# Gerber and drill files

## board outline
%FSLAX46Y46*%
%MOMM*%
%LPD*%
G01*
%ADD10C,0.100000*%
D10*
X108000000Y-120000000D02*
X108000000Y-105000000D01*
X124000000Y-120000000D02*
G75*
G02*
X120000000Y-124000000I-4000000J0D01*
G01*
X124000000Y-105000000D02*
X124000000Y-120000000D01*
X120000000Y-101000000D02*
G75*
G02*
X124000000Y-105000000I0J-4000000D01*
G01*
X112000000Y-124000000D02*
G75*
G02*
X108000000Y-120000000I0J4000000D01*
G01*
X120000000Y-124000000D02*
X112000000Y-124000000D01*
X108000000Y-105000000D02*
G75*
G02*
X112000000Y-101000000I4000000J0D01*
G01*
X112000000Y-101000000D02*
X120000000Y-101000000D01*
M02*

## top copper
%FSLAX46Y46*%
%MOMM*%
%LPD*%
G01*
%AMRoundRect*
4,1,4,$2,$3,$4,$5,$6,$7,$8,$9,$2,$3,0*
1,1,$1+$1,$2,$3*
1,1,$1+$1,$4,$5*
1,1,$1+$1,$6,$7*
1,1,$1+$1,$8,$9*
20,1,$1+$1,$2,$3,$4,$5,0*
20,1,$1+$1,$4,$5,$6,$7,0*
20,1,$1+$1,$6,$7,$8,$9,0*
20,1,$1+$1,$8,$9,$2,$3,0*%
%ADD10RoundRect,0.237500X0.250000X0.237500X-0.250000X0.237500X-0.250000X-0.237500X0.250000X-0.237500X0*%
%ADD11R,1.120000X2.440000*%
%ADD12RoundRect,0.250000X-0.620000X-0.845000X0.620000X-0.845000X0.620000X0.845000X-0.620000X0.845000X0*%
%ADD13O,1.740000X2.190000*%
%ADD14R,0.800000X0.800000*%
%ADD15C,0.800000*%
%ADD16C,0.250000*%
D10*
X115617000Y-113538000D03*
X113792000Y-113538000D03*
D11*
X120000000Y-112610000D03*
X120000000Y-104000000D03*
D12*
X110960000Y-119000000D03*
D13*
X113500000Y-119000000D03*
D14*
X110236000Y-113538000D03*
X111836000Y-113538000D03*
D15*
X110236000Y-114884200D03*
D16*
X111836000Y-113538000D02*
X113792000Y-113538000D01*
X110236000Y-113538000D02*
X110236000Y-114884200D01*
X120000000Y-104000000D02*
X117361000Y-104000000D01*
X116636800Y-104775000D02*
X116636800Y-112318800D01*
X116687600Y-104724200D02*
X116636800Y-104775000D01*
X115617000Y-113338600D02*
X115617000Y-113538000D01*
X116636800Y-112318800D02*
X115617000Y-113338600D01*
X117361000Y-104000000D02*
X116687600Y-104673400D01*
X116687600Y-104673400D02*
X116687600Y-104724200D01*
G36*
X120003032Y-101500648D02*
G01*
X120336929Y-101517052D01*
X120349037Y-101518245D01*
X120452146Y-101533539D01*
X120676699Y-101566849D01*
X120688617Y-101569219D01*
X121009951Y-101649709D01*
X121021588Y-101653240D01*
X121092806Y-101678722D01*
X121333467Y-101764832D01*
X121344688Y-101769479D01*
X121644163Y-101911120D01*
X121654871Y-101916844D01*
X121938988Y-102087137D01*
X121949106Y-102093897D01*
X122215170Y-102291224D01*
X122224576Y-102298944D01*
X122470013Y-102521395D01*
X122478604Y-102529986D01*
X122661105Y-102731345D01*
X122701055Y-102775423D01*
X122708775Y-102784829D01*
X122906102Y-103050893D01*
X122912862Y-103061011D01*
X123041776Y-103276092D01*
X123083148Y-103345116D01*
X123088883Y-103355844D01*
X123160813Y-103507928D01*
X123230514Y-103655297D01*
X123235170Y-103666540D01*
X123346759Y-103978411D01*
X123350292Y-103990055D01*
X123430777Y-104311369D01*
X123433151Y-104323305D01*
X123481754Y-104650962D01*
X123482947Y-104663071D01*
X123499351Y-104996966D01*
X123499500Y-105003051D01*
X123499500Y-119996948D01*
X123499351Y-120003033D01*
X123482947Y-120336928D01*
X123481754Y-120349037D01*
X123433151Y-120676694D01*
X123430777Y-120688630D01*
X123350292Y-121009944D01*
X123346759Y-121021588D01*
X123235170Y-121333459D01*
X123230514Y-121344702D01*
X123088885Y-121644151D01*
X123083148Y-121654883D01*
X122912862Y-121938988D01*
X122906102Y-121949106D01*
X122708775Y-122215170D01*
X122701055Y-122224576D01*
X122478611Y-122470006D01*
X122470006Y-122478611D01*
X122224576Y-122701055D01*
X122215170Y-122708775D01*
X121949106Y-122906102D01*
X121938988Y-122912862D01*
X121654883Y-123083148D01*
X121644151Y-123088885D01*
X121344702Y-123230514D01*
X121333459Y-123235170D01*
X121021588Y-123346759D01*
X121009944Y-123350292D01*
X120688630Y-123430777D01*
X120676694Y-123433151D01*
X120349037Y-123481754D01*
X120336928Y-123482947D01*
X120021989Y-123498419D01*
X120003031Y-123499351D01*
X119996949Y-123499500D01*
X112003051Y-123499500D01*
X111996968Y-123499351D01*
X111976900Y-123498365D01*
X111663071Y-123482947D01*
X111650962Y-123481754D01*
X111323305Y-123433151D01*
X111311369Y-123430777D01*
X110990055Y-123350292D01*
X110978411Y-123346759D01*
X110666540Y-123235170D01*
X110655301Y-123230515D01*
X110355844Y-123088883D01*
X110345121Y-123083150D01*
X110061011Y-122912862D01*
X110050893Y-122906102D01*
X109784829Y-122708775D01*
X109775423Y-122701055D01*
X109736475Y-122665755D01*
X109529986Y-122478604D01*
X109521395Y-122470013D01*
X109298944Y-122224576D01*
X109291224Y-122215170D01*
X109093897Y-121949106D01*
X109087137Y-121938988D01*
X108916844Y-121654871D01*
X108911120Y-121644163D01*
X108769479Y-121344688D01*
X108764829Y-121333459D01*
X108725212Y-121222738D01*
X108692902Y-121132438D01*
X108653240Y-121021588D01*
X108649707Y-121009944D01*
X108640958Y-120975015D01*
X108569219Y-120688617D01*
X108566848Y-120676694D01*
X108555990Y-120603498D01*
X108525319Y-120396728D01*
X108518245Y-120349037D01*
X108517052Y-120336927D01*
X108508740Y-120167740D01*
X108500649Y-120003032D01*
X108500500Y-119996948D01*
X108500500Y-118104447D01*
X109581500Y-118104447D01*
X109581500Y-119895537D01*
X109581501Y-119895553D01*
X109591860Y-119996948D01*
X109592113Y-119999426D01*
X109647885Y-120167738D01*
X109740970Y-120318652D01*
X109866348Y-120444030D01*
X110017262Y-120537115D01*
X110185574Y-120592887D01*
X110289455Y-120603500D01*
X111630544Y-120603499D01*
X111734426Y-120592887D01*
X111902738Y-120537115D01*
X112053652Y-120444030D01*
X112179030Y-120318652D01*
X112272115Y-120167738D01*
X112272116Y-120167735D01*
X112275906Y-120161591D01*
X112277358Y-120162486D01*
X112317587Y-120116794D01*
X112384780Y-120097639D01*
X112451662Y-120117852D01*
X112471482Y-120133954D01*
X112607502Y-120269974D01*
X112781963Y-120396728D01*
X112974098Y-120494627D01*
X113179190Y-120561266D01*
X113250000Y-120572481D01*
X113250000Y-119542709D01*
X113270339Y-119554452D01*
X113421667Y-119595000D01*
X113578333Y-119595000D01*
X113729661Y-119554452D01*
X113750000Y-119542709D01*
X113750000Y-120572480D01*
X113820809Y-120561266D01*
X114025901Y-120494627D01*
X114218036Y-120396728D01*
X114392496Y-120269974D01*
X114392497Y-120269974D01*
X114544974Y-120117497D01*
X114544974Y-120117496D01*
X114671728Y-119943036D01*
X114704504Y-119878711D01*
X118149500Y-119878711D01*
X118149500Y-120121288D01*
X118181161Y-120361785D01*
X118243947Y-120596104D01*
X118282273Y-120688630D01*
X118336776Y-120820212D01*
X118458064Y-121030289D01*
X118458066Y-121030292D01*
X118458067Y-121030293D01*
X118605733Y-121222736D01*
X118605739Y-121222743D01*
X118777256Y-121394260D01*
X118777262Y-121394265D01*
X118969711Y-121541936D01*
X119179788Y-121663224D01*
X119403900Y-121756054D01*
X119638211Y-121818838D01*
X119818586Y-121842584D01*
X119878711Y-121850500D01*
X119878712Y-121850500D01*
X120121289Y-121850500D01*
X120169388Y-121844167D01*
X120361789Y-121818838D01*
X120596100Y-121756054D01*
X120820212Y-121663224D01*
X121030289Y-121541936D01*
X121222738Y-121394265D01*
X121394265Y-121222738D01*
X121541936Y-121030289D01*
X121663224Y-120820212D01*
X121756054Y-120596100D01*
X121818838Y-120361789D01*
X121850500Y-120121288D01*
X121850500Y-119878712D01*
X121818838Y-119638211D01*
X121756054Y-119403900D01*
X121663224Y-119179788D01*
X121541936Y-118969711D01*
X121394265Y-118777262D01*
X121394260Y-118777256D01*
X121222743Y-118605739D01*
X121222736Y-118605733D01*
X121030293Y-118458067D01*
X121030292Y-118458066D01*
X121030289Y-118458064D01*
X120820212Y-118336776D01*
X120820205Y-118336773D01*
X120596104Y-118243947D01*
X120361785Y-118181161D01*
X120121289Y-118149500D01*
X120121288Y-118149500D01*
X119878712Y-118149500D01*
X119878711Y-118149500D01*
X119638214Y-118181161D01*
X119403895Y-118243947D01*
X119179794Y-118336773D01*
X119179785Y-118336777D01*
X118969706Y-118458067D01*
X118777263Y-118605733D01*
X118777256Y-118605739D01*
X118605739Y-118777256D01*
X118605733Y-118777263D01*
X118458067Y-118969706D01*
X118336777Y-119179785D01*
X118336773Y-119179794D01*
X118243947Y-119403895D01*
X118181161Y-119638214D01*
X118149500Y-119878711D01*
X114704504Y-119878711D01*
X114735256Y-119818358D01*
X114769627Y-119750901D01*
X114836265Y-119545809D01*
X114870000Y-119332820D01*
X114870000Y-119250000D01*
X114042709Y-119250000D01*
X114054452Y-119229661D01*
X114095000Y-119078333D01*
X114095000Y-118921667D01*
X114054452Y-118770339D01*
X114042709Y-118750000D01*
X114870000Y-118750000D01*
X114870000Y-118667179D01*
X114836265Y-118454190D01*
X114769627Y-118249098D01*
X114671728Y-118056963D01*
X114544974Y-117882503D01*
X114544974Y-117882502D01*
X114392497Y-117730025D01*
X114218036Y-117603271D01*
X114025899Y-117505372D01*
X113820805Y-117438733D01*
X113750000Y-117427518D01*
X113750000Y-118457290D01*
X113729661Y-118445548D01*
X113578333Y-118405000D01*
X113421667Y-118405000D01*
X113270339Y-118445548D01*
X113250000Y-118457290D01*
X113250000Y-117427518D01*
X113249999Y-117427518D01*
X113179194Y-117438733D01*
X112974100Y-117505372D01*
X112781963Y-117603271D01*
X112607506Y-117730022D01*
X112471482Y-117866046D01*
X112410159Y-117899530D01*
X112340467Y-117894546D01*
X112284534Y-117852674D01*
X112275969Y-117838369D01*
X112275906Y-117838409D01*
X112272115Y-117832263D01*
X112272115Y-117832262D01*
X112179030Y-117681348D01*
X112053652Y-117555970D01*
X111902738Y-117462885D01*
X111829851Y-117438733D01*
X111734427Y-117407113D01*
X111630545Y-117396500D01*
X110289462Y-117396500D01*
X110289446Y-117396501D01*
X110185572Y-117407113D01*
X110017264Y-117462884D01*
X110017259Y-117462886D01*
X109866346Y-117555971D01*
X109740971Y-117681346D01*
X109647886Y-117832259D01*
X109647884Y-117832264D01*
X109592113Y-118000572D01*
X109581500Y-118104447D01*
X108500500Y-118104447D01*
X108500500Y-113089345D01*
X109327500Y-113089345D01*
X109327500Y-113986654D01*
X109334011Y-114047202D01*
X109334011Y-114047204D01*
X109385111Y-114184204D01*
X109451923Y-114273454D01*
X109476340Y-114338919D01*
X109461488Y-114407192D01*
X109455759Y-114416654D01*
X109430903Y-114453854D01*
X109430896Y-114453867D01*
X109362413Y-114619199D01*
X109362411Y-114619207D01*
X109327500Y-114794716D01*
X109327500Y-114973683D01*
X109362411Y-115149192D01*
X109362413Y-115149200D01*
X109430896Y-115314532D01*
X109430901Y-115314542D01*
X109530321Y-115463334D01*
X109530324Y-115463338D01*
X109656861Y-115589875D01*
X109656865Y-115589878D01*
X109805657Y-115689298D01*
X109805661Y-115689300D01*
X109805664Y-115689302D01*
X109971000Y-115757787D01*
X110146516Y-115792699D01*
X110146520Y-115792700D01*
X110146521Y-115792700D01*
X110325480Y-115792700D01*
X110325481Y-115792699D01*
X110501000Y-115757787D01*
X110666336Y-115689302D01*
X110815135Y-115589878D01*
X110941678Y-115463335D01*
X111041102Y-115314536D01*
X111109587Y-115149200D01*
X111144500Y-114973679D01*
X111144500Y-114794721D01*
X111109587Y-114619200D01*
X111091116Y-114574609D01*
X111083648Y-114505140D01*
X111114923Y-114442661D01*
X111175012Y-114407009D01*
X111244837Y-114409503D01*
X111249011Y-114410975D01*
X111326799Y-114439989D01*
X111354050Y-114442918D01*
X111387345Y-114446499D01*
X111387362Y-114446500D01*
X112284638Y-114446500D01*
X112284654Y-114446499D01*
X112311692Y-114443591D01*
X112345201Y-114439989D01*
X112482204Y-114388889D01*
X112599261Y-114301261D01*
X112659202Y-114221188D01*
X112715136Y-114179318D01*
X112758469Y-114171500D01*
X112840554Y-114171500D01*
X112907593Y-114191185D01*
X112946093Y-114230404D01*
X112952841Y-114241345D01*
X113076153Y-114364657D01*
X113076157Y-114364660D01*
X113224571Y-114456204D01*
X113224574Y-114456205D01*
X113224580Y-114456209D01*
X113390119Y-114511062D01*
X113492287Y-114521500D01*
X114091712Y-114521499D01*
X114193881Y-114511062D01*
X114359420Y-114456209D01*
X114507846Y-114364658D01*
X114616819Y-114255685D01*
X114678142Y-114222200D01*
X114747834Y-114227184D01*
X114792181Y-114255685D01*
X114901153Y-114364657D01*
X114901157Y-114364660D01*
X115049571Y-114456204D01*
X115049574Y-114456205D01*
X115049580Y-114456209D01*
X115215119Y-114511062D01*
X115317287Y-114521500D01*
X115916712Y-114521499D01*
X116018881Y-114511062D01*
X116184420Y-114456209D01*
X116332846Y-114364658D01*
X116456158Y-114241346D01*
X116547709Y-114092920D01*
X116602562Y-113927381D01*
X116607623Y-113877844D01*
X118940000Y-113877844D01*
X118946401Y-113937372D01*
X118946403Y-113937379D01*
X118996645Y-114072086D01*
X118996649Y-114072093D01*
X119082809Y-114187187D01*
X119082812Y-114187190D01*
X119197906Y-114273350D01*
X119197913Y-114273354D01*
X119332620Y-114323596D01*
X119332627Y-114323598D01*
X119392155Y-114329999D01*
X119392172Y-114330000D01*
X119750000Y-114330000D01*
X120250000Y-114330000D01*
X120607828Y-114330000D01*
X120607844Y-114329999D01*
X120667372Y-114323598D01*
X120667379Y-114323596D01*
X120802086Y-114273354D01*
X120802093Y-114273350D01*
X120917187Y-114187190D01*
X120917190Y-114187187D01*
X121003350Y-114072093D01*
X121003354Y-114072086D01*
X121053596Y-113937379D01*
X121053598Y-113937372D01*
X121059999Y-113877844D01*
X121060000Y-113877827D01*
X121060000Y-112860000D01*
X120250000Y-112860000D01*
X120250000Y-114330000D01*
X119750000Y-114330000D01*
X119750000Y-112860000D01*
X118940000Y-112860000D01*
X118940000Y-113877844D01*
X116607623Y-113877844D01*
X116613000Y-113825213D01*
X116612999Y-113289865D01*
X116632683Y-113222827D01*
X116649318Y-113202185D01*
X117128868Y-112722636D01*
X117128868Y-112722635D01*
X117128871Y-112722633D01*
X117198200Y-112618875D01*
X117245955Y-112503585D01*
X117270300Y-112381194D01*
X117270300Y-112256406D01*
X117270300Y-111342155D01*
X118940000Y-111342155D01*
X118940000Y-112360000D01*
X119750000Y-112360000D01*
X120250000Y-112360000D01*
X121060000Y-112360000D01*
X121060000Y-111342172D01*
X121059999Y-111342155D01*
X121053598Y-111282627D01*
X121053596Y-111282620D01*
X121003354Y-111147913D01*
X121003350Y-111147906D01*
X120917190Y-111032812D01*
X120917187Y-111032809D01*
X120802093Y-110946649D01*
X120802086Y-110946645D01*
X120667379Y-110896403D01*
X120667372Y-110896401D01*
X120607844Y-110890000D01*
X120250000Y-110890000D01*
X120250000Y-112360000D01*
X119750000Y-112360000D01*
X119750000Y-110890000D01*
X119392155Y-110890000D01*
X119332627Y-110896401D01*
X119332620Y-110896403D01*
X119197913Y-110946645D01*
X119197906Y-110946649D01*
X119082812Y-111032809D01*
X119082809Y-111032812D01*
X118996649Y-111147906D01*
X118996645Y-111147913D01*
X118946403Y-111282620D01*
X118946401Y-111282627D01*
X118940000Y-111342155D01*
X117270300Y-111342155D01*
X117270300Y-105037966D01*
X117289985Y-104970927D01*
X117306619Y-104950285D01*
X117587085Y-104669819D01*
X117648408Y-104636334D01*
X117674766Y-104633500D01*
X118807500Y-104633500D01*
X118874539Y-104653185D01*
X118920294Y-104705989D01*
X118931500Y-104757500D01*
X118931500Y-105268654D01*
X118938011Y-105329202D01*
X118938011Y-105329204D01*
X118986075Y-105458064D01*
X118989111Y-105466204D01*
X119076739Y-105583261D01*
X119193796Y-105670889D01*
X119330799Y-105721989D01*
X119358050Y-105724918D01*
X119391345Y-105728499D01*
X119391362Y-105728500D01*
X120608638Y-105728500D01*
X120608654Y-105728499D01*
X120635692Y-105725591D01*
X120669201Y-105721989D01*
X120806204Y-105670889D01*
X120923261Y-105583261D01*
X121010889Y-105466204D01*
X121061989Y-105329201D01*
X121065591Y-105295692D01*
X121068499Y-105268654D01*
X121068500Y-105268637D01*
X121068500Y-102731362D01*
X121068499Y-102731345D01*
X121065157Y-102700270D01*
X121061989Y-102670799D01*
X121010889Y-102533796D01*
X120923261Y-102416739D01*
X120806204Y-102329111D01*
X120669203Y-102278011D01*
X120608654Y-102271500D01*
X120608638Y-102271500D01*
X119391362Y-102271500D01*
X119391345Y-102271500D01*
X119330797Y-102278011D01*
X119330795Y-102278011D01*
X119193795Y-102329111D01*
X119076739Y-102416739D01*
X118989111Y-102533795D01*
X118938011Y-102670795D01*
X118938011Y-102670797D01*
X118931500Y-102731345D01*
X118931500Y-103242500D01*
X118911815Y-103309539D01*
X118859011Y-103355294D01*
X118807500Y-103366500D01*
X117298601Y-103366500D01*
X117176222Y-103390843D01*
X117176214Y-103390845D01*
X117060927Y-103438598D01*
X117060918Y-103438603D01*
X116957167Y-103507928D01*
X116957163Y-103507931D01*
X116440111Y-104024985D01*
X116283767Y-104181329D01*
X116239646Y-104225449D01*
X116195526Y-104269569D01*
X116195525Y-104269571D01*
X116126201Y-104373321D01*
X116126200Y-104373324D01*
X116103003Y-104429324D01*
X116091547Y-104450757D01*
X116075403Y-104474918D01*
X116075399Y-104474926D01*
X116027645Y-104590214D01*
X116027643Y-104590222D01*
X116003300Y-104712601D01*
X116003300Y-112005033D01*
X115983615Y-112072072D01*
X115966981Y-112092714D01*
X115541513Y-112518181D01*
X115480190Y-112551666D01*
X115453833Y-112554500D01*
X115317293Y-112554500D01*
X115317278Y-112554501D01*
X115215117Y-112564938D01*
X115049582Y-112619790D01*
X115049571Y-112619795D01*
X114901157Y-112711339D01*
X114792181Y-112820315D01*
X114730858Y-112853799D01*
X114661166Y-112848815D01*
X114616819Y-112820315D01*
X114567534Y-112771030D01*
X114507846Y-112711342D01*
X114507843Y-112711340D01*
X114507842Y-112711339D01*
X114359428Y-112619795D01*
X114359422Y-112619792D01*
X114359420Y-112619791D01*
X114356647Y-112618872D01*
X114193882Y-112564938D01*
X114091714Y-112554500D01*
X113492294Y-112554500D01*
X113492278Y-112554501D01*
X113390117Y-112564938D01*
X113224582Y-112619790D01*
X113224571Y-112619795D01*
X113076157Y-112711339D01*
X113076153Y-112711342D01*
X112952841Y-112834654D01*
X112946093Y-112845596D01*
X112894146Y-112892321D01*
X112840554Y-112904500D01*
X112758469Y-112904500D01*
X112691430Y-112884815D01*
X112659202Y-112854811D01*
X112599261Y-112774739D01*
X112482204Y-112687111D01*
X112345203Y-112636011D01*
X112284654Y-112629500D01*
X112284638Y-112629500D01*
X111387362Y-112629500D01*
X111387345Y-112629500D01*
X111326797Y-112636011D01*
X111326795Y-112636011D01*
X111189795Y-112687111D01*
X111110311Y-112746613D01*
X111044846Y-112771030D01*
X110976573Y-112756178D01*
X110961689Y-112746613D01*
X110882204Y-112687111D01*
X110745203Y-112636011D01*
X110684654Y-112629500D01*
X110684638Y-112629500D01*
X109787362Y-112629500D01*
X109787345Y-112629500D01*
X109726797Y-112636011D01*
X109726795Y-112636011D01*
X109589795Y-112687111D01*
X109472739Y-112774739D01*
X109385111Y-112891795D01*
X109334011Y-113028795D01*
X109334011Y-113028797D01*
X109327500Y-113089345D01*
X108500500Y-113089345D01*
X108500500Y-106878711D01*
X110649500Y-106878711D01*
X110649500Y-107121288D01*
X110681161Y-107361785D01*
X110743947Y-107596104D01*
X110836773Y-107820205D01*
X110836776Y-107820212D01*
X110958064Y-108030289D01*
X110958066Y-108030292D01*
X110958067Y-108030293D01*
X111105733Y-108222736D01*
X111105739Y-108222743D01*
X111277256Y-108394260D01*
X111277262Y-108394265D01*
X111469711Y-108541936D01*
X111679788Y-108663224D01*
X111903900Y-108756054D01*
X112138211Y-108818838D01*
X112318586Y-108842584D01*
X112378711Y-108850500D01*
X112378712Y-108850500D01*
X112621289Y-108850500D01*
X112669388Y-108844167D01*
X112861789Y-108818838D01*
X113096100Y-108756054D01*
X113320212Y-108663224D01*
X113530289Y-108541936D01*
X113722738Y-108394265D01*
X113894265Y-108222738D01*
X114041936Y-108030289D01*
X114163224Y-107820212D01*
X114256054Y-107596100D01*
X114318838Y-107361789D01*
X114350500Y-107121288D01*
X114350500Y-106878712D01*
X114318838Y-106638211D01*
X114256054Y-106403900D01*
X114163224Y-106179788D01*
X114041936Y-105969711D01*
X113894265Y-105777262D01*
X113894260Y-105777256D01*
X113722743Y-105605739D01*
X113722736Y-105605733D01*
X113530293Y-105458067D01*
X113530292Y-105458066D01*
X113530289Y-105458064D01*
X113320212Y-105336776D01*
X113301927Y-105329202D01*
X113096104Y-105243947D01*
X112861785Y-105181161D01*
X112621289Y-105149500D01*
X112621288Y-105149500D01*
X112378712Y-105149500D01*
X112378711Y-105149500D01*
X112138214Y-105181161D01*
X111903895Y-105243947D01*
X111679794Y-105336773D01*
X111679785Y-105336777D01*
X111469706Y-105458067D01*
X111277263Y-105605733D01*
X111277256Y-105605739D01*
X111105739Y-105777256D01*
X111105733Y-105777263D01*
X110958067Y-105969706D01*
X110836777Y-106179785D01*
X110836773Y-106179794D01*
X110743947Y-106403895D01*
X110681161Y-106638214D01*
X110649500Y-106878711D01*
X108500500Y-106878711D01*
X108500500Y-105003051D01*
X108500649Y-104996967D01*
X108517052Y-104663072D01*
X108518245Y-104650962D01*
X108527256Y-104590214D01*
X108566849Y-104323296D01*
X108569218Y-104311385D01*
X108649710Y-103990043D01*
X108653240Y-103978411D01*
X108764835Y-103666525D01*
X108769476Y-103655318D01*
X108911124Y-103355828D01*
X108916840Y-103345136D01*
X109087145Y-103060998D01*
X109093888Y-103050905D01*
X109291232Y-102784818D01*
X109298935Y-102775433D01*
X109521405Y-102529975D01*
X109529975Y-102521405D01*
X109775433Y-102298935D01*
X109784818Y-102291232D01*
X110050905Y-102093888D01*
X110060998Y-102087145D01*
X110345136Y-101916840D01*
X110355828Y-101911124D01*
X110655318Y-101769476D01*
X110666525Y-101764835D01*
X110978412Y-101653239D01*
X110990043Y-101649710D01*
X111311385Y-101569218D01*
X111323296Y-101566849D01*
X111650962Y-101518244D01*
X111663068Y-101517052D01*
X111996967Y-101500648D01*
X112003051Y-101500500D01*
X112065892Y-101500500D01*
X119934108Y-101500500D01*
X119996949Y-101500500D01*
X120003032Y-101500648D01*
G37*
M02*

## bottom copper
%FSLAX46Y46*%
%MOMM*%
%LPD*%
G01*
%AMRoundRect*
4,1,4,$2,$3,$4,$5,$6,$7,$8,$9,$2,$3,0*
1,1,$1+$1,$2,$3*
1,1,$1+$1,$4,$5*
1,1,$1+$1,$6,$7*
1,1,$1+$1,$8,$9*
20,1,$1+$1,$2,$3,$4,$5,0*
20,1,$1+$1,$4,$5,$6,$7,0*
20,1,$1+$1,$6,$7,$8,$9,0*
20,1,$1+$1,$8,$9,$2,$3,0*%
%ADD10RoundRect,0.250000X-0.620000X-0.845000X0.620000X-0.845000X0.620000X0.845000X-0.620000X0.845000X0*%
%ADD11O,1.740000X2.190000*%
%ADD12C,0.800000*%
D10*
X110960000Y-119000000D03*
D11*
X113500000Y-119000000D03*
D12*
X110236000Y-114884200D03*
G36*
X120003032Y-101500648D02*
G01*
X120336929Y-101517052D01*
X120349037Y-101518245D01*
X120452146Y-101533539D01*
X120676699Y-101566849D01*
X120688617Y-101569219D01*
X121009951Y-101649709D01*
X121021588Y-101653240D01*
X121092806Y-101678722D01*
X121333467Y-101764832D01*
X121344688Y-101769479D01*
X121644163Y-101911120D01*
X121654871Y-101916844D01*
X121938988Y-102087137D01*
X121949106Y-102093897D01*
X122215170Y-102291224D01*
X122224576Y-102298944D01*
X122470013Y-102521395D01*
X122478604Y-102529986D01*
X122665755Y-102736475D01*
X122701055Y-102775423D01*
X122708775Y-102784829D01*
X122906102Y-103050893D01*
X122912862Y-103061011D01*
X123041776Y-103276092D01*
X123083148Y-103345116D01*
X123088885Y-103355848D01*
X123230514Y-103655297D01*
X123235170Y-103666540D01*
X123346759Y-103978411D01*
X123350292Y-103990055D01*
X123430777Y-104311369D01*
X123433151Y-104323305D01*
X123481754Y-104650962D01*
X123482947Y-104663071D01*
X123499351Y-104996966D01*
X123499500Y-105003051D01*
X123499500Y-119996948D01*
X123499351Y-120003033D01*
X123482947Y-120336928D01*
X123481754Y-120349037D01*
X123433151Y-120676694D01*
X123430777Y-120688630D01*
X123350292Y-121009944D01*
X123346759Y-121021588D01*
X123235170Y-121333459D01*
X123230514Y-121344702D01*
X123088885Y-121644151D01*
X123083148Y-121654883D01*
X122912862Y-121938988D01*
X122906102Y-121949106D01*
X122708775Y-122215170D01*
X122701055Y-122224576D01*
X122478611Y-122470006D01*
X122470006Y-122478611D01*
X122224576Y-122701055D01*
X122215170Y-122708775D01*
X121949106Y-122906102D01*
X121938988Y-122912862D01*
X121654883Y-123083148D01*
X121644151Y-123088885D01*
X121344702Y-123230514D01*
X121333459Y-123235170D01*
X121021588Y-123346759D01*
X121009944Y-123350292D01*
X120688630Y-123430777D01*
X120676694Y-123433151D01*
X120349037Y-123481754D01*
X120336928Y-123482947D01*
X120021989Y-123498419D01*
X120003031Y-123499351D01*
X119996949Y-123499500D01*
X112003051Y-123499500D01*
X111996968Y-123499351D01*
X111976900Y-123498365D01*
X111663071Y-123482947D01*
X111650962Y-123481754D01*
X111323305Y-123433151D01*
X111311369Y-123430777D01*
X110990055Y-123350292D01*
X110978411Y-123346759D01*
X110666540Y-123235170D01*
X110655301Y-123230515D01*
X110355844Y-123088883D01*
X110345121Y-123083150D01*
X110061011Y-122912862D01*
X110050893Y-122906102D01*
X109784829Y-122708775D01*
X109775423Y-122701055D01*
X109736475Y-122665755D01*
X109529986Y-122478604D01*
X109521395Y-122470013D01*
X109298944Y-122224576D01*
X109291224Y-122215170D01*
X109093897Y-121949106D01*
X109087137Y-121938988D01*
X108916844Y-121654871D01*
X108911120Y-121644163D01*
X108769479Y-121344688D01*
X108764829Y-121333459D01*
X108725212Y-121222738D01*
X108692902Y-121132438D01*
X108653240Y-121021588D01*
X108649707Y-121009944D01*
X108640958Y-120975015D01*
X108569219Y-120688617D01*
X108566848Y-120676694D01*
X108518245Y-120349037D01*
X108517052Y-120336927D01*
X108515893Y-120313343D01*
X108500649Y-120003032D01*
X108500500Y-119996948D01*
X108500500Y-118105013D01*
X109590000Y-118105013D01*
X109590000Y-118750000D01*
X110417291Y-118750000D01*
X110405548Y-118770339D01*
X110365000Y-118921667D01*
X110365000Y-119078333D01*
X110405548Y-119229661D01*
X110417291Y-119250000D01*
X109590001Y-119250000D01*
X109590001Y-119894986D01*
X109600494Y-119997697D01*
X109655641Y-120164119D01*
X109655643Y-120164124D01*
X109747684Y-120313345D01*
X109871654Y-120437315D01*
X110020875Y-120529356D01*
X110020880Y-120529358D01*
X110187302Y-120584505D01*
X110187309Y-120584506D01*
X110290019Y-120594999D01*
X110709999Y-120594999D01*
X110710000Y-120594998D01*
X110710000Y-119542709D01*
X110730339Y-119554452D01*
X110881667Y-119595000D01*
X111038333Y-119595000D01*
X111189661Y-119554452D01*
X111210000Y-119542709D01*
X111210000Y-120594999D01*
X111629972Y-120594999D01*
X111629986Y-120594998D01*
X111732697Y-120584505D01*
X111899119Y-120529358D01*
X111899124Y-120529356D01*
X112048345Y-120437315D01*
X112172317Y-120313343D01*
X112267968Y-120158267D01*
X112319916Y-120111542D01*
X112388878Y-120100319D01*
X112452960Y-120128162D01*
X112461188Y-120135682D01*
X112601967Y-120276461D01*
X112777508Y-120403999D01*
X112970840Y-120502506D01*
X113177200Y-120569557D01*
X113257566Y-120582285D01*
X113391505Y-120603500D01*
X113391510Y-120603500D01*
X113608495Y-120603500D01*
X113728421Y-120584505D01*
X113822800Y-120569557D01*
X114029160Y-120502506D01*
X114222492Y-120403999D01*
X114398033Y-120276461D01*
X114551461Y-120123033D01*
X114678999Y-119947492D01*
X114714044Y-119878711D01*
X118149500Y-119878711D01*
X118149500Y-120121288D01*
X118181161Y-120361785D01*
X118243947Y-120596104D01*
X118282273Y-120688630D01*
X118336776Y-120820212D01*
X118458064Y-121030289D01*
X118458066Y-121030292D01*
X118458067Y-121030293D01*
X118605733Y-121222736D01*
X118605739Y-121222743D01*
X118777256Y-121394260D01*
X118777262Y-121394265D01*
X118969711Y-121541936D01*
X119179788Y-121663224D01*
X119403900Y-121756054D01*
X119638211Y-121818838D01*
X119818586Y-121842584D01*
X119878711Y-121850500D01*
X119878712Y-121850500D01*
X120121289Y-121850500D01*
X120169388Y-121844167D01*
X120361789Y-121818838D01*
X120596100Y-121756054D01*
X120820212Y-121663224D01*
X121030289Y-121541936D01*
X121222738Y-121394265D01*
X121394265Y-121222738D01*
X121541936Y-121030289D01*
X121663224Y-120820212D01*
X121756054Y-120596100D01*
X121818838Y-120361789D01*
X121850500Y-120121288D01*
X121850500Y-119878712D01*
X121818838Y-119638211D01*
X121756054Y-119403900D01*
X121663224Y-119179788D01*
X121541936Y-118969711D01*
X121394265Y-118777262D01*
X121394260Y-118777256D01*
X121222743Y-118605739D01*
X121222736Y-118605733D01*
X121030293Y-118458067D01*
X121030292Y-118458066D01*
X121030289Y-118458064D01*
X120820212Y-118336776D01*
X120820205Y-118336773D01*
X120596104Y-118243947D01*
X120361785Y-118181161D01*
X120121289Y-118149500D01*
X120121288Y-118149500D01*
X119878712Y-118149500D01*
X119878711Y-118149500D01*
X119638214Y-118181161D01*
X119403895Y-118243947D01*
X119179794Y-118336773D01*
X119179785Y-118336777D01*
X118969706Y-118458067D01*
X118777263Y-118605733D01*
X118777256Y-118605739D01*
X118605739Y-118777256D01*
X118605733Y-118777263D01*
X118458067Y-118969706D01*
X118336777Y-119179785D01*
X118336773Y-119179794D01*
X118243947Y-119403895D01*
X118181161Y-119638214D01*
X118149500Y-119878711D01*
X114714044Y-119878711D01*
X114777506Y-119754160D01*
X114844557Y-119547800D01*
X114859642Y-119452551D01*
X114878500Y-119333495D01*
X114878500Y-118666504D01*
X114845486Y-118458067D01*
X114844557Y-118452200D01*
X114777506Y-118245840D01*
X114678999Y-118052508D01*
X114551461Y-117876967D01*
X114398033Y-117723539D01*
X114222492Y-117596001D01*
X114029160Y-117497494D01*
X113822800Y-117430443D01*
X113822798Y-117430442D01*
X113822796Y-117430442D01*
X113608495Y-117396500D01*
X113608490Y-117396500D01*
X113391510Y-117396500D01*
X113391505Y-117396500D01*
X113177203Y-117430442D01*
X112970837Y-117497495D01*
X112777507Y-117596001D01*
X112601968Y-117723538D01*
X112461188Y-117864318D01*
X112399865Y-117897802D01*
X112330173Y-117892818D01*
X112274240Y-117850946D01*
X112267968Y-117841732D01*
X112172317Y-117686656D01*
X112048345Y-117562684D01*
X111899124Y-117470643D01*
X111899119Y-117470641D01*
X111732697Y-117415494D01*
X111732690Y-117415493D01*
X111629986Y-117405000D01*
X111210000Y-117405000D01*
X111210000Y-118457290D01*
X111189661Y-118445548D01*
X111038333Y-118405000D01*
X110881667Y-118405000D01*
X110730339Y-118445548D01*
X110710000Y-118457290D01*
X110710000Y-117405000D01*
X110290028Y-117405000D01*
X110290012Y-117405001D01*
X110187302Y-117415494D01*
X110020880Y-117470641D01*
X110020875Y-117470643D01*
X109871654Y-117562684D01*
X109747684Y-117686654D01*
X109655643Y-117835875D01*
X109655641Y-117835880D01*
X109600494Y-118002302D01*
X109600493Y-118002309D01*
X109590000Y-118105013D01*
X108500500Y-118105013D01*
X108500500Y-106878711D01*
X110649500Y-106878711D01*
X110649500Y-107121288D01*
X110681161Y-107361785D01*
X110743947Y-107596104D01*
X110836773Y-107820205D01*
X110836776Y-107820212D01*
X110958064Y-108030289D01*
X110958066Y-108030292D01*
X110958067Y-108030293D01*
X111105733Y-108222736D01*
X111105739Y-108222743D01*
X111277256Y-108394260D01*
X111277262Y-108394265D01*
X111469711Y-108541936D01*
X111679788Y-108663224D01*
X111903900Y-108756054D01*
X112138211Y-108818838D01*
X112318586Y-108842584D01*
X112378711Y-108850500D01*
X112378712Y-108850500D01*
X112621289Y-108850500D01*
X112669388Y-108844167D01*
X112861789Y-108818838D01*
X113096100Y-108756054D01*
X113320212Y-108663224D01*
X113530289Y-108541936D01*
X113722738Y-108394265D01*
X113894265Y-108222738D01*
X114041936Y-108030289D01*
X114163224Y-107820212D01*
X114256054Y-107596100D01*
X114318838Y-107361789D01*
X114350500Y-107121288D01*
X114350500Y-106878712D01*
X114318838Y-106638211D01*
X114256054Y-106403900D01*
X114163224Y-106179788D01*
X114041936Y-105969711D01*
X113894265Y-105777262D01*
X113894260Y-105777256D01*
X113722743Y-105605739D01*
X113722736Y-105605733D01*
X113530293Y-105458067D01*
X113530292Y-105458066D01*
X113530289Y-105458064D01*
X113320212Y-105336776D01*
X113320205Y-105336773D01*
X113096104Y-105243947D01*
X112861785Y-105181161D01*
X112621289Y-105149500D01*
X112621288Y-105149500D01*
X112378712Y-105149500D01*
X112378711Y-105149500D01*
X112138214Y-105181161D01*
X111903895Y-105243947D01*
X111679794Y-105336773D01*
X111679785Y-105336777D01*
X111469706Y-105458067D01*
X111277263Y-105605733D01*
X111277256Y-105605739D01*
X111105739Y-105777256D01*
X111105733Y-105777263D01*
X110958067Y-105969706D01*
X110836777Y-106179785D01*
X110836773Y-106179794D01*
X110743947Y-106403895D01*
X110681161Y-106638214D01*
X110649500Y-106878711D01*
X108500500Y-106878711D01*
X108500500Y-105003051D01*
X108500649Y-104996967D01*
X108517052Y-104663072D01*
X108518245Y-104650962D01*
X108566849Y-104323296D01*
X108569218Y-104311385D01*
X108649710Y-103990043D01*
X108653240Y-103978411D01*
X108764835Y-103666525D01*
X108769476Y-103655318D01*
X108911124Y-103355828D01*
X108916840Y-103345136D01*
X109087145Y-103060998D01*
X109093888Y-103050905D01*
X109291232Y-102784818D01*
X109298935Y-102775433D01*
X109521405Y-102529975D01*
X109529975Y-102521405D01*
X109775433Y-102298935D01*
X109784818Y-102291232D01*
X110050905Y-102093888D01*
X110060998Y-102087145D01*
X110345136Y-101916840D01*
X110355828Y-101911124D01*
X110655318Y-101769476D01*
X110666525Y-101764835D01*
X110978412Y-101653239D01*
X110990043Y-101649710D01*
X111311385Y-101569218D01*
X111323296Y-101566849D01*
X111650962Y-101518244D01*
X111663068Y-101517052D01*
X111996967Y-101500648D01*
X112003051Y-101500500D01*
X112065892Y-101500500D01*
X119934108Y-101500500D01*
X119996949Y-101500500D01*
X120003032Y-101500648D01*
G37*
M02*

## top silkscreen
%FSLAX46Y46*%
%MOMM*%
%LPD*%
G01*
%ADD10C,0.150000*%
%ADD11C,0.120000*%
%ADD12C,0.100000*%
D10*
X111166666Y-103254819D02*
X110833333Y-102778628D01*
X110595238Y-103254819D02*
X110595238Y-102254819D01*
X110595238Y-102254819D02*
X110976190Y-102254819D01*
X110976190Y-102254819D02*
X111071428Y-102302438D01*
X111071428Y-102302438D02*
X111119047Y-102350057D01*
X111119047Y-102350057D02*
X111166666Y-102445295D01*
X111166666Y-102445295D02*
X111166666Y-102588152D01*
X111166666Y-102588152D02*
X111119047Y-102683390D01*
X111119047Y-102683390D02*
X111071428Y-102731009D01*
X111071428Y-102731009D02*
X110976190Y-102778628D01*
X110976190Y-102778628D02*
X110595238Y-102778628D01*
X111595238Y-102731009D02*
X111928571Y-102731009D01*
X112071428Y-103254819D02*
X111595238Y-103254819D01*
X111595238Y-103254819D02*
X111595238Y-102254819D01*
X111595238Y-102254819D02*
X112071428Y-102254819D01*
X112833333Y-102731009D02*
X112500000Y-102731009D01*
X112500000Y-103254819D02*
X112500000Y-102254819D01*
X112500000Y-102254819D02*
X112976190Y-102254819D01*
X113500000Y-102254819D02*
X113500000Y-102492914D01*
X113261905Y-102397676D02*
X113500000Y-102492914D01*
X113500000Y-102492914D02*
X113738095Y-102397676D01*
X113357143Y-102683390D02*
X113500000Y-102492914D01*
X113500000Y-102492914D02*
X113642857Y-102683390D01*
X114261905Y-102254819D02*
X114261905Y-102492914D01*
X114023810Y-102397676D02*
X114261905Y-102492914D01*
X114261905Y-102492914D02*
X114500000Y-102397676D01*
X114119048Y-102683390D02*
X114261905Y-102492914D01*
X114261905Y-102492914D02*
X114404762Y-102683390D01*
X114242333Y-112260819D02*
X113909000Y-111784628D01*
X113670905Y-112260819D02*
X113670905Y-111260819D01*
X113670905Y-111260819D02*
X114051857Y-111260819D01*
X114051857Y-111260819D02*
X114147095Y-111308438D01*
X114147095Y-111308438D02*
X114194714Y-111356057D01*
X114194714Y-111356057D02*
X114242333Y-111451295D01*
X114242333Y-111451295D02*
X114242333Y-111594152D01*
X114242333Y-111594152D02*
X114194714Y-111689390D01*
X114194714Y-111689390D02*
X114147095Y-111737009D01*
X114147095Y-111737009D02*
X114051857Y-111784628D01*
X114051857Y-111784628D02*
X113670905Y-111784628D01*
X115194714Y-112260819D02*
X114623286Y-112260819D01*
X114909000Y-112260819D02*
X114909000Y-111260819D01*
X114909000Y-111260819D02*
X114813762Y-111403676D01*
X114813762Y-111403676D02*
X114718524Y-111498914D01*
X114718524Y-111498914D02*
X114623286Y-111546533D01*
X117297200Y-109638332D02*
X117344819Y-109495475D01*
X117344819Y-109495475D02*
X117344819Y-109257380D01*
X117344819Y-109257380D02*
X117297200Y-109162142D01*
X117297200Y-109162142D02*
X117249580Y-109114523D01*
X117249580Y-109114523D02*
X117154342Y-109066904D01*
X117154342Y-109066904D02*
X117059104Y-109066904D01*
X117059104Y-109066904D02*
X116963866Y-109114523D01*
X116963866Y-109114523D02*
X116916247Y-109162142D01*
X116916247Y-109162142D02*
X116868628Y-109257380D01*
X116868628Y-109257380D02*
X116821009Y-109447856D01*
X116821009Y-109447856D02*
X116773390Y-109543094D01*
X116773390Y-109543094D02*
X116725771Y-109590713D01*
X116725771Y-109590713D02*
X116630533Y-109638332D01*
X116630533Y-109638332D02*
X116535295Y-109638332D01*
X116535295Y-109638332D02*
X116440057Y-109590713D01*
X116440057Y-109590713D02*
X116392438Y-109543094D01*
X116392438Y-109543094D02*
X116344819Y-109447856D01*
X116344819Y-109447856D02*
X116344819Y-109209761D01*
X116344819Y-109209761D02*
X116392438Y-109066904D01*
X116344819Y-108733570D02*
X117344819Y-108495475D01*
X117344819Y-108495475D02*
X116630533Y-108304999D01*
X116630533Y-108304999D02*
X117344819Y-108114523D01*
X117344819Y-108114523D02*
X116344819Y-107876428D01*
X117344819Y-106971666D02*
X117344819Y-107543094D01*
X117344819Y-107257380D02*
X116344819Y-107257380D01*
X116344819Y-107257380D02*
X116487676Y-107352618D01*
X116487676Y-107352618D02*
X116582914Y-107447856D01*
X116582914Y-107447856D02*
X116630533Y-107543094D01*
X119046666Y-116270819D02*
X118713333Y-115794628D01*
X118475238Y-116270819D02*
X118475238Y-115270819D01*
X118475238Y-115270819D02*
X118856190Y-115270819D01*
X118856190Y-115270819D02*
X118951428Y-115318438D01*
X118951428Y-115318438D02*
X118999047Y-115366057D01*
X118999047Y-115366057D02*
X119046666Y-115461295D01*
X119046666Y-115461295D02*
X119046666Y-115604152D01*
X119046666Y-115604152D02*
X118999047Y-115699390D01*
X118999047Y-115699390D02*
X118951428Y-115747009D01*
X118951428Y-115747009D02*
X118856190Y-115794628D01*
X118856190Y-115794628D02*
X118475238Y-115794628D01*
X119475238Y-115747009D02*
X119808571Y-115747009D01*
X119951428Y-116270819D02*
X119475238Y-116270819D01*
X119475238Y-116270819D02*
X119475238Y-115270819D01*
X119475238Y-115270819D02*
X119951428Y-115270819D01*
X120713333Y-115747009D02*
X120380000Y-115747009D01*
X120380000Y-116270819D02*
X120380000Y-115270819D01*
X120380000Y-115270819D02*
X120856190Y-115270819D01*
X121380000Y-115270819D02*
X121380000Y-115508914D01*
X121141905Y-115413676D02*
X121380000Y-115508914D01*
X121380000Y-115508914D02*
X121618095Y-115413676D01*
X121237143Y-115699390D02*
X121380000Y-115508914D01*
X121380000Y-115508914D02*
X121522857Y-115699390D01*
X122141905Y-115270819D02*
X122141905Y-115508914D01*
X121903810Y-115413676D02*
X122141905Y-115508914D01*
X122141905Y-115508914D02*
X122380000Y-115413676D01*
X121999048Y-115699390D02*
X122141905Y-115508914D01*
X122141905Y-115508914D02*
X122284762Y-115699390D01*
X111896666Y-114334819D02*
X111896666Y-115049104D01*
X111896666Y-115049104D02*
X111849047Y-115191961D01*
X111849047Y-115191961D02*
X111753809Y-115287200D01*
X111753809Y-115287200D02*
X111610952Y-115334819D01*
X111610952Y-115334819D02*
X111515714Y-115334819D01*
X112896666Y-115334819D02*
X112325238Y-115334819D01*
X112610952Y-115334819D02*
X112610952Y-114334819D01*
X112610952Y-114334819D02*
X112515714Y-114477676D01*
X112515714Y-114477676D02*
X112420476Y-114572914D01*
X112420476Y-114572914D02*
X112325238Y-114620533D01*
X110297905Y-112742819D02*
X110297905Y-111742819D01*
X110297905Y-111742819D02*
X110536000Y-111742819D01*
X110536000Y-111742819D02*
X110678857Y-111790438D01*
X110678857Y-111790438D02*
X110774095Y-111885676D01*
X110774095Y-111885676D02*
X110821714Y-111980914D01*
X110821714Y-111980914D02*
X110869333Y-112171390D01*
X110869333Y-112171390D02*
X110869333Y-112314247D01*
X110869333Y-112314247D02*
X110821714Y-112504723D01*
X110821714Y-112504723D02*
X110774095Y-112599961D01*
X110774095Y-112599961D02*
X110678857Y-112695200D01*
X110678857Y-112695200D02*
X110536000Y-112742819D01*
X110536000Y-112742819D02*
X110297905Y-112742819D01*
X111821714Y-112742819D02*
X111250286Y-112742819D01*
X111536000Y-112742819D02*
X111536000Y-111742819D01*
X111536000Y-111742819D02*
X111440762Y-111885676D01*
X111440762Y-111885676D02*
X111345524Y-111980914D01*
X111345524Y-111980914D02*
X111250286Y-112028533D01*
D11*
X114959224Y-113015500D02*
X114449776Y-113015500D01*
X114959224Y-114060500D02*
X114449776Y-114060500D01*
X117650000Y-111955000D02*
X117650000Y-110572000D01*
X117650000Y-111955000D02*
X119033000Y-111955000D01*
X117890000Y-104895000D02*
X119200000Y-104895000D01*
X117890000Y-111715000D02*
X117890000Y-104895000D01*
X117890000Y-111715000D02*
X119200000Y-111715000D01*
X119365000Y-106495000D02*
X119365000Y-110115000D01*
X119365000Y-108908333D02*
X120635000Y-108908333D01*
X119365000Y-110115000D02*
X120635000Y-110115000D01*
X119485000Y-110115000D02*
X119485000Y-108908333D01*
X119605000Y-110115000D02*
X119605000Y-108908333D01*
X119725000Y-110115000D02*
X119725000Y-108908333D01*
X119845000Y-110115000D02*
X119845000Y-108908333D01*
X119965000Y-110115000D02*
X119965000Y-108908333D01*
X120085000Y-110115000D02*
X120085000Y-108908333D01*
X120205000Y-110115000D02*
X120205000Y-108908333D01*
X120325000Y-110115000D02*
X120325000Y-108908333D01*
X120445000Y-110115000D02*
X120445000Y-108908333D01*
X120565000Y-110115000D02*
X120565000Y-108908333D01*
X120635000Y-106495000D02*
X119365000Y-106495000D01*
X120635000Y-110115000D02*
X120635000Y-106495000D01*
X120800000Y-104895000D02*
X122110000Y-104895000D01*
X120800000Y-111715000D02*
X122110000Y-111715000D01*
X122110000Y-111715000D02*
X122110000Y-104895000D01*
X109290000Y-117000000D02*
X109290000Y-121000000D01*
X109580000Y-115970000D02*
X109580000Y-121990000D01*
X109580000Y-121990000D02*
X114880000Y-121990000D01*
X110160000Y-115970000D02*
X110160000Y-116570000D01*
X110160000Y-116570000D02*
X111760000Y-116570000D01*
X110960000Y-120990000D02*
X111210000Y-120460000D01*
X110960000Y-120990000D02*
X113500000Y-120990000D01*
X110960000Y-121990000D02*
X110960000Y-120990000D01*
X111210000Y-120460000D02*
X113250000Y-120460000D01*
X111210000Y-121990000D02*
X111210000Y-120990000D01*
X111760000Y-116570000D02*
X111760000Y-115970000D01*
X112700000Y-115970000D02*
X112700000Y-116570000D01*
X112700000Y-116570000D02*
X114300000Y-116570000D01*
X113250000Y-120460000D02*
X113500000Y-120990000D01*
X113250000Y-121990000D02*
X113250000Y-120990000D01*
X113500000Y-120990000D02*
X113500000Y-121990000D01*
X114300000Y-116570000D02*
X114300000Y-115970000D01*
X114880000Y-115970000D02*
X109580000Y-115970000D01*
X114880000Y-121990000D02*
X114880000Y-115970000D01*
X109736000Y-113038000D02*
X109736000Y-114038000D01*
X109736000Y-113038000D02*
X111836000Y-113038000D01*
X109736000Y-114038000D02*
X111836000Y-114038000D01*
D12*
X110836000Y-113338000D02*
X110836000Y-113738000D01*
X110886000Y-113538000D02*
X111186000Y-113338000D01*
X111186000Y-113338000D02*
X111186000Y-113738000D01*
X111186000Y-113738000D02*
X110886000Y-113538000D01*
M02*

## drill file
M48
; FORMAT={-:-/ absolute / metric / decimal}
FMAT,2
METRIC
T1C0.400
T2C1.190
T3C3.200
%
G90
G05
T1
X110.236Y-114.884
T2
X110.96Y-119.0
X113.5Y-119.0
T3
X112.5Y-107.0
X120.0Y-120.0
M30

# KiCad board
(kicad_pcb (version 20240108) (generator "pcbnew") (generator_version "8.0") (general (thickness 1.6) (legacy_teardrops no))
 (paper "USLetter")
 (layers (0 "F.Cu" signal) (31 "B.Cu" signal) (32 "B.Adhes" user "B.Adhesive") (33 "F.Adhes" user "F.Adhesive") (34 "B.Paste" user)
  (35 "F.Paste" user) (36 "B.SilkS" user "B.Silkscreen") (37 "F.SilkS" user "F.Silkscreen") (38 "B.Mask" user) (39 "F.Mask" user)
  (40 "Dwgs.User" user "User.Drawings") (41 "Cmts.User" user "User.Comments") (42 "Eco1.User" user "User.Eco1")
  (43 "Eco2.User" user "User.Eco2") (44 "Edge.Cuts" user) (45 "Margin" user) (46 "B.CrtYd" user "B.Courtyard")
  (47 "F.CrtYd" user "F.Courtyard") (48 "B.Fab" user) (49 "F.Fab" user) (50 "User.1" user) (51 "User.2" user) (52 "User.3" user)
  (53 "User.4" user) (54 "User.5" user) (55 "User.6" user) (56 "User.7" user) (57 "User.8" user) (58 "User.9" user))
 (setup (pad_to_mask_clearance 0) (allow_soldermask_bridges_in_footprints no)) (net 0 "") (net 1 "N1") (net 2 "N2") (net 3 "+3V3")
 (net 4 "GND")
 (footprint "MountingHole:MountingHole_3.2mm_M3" (layer "F.Cu") (at 112.5 107)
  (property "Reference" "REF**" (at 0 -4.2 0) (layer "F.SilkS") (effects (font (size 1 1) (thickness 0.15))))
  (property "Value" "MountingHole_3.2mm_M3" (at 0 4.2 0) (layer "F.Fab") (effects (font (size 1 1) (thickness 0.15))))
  (pad "" np_thru_hole circle (at 0 0) (size 3.2 3.2) (drill 3.2) (layers "*.Cu" "*.Mask")))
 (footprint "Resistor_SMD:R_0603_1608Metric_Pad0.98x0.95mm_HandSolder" (layer "F.Cu") (at 114.7045 113.538 180)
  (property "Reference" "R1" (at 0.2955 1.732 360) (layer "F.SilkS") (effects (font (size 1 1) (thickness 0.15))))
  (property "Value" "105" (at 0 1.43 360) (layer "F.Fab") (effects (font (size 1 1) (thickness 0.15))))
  (fp_line (start -0.254724 0.5225) (end 0.254724 0.5225) (stroke (width 0.12) (type solid)) (layer "F.SilkS"))
  (fp_line (start -0.254724 -0.5225) (end 0.254724 -0.5225) (stroke (width 0.12) (type solid)) (layer "F.SilkS"))
  (pad "1" smd roundrect (at -0.9125 0 180) (size 0.975 0.95) (layers "F.Cu" "F.Paste" "F.Mask") (roundrect_rratio 0.25) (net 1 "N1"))
  (pad "2" smd roundrect (at 0.9125 0 180) (size 0.975 0.95) (layers "F.Cu" "F.Paste" "F.Mask") (roundrect_rratio 0.25) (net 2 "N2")))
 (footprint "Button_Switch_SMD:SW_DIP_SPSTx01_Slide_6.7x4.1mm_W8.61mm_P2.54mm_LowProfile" (layer "F.Cu") (at 120 108.305 90)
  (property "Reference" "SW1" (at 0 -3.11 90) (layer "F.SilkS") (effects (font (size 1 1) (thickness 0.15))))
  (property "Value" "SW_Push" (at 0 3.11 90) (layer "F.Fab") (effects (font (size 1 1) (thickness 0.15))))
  (fp_line (start -3.65 -2.35) (end -2.267 -2.35) (stroke (width 0.12) (type solid)) (layer "F.SilkS"))
  (fp_line (start -3.65 -2.35) (end -3.65 -0.967) (stroke (width 0.12) (type solid)) (layer "F.SilkS"))
  (fp_line (start 3.41 -2.11) (end 3.41 -0.8) (stroke (width 0.12) (type solid)) (layer "F.SilkS"))
  (fp_line (start -3.41 -2.11) (end 3.41 -2.11) (stroke (width 0.12) (type solid)) (layer "F.SilkS"))
  (fp_line (start -3.41 -2.11) (end -3.41 -0.8) (stroke (width 0.12) (type solid)) (layer "F.SilkS"))
  (fp_line (start 1.81 -0.635) (end -1.81 -0.635) (stroke (width 0.12) (type solid)) (layer "F.SilkS"))
  (fp_line (start -0.603333 -0.635) (end -0.603333 0.635) (stroke (width 0.12) (type solid)) (layer "F.SilkS"))
  (fp_line (start -1.81 -0.635) (end -1.81 0.635) (stroke (width 0.12) (type solid)) (layer "F.SilkS"))
  (fp_line (start -1.81 -0.515) (end -0.603333 -0.515) (stroke (width 0.12) (type solid)) (layer "F.SilkS"))
  (fp_line (start -1.81 -0.395) (end -0.603333 -0.395) (stroke (width 0.12) (type solid)) (layer "F.SilkS"))
  (fp_line (start -1.81 -0.275) (end -0.603333 -0.275) (stroke (width 0.12) (type solid)) (layer "F.SilkS"))
  (fp_line (start -1.81 -0.155) (end -0.603333 -0.155) (stroke (width 0.12) (type solid)) (layer "F.SilkS"))
  (fp_line (start -1.81 -0.035) (end -0.603333 -0.035) (stroke (width 0.12) (type solid)) (layer "F.SilkS"))
  (fp_line (start -1.81 0.085) (end -0.603333 0.085) (stroke (width 0.12) (type solid)) (layer "F.SilkS"))
  (fp_line (start -1.81 0.205) (end -0.603333 0.205) (stroke (width 0.12) (type solid)) (layer "F.SilkS"))
  (fp_line (start -1.81 0.325) (end -0.603333 0.325) (stroke (width 0.12) (type solid)) (layer "F.SilkS"))
  (fp_line (start -1.81 0.445) (end -0.603333 0.445) (stroke (width 0.12) (type solid)) (layer "F.SilkS"))
  (fp_line (start -1.81 0.565) (end -0.603333 0.565) (stroke (width 0.12) (type solid)) (layer "F.SilkS"))
  (fp_line (start 1.81 0.635) (end 1.81 -0.635) (stroke (width 0.12) (type solid)) (layer "F.SilkS"))
  (fp_line (start -1.81 0.635) (end 1.81 0.635) (stroke (width 0.12) (type solid)) (layer "F.SilkS"))
  (fp_line (start 3.41 0.8) (end 3.41 2.11) (stroke (width 0.12) (type solid)) (layer "F.SilkS"))
  (fp_line (start -3.41 0.8) (end -3.41 2.11) (stroke (width 0.12) (type solid)) (layer "F.SilkS"))
  (fp_line (start -3.41 2.11) (end 3.41 2.11) (stroke (width 0.12) (type solid)) (layer "F.SilkS"))
  (pad "1" smd rect (at -4.305 0 90) (size 2.44 1.12) (layers "F.Cu" "F.Paste" "F.Mask") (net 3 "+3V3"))
  (pad "2" smd rect (at 4.305 0 90) (size 2.44 1.12) (layers "F.Cu" "F.Paste" "F.Mask") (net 1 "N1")))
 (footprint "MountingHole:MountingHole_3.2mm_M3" (layer "F.Cu") (at 120 120)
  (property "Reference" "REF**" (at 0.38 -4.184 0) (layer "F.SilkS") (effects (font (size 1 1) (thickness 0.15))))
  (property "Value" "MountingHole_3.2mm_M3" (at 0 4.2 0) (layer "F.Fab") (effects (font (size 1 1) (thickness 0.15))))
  (pad "" np_thru_hole circle (at 0 0) (size 3.2 3.2) (drill 3.2) (layers "*.Cu" "*.Mask")))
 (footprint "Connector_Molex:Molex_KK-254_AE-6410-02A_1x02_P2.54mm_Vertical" (layer "F.Cu") (at 110.96 119)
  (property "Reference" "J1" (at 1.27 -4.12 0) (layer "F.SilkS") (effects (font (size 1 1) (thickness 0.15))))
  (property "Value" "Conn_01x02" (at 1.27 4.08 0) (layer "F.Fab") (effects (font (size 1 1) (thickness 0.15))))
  (fp_line (start -1.67 -2) (end -1.67 2) (stroke (width 0.12) (type solid)) (layer "F.SilkS"))
  (fp_line (start -1.38 -3.03) (end -1.38 2.99) (stroke (width 0.12) (type solid)) (layer "F.SilkS"))
  (fp_line (start -1.38 2.99) (end 3.92 2.99) (stroke (width 0.12) (type solid)) (layer "F.SilkS"))
  (fp_line (start -0.8 -3.03) (end -0.8 -2.43) (stroke (width 0.12) (type solid)) (layer "F.SilkS"))
  (fp_line (start -0.8 -2.43) (end 0.8 -2.43) (stroke (width 0.12) (type solid)) (layer "F.SilkS"))
  (fp_line (start 0 1.99) (end 0.25 1.46) (stroke (width 0.12) (type solid)) (layer "F.SilkS"))
  (fp_line (start 0 1.99) (end 2.54 1.99) (stroke (width 0.12) (type solid)) (layer "F.SilkS"))
  (fp_line (start 0 2.99) (end 0 1.99) (stroke (width 0.12) (type solid)) (layer "F.SilkS"))
  (fp_line (start 0.25 1.46) (end 2.29 1.46) (stroke (width 0.12) (type solid)) (layer "F.SilkS"))
  (fp_line (start 0.25 2.99) (end 0.25 1.99) (stroke (width 0.12) (type solid)) (layer "F.SilkS"))
  (fp_line (start 0.8 -2.43) (end 0.8 -3.03) (stroke (width 0.12) (type solid)) (layer "F.SilkS"))
  (fp_line (start 1.74 -3.03) (end 1.74 -2.43) (stroke (width 0.12) (type solid)) (layer "F.SilkS"))
  (fp_line (start 1.74 -2.43) (end 3.34 -2.43) (stroke (width 0.12) (type solid)) (layer "F.SilkS"))
  (fp_line (start 2.29 1.46) (end 2.54 1.99) (stroke (width 0.12) (type solid)) (layer "F.SilkS"))
  (fp_line (start 2.29 2.99) (end 2.29 1.99) (stroke (width 0.12) (type solid)) (layer "F.SilkS"))
  (fp_line (start 2.54 1.99) (end 2.54 2.99) (stroke (width 0.12) (type solid)) (layer "F.SilkS"))
  (fp_line (start 3.34 -2.43) (end 3.34 -3.03) (stroke (width 0.12) (type solid)) (layer "F.SilkS"))
  (fp_line (start 3.92 -3.03) (end -1.38 -3.03) (stroke (width 0.12) (type solid)) (layer "F.SilkS"))
  (fp_line (start 3.92 2.99) (end 3.92 -3.03) (stroke (width 0.12) (type solid)) (layer "F.SilkS"))
  (pad "1" thru_hole roundrect (at 0 0) (size 1.74 2.19) (drill 1.19) (layers "*.Cu" "*.Mask") (remove_unused_layers no)
   (roundrect_rratio 0.143678) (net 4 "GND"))
  (pad "2" thru_hole oval (at 2.54 0) (size 1.74 2.19) (drill 1.19) (layers "*.Cu" "*.Mask") (remove_unused_layers no) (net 3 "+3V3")))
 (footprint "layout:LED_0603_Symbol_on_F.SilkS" (layer "F.Cu") (at 111.036 113.538)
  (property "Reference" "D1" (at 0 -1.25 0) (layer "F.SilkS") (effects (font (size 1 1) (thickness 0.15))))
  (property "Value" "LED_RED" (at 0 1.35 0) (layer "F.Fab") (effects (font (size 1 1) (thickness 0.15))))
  (fp_line (start -1.3 -0.5) (end -1.3 0.5) (stroke (width 0.12) (type solid)) (layer "F.SilkS"))
  (fp_line (start -1.3 -0.5) (end 0.8 -0.5) (stroke (width 0.12) (type solid)) (layer "F.SilkS"))
  (fp_line (start -1.3 0.5) (end 0.8 0.5) (stroke (width 0.12) (type solid)) (layer "F.SilkS"))
  (fp_line (start -0.2 -0.2) (end -0.2 0.2) (stroke (width 0.1) (type solid)) (layer "F.SilkS"))
  (fp_line (start -0.15 0) (end 0.15 -0.2) (stroke (width 0.1) (type solid)) (layer "F.SilkS"))
  (fp_line (start 0.15 -0.2) (end 0.15 0.2) (stroke (width 0.1) (type solid)) (layer "F.SilkS"))
  (fp_line (start 0.15 0.2) (end -0.15 0) (stroke (width 0.1) (type solid)) (layer "F.SilkS"))
  (pad "1" smd rect (at -0.8 0 180) (size 0.8 0.8) (layers "F.Cu" "F.Paste" "F.Mask") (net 4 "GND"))
  (pad "2" smd rect (at 0.8 0 180) (size 0.8 0.8) (layers "F.Cu" "F.Paste" "F.Mask") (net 2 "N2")))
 (gr_line (start 108 120) (end 108 105) (stroke (width 0.1) (type default)) (layer "Edge.Cuts"))
 (gr_arc (start 124 120) (mid 122.828427 122.828427) (end 120 124) (stroke (width 0.1) (type default)) (layer "Edge.Cuts"))
 (gr_line (start 124 105) (end 124 120) (stroke (width 0.1) (type default)) (layer "Edge.Cuts"))
 (gr_arc (start 120 101) (mid 122.828427 102.171573) (end 124 105) (stroke (width 0.1) (type default)) (layer "Edge.Cuts"))
 (gr_arc (start 112 124) (mid 109.171573 122.828427) (end 108 120) (stroke (width 0.1) (type default)) (layer "Edge.Cuts"))
 (gr_line (start 120 124) (end 112 124) (stroke (width 0.1) (type default)) (layer "Edge.Cuts"))
 (gr_arc (start 108 105) (mid 109.171573 102.171573) (end 112 101) (stroke (width 0.1) (type default)) (layer "Edge.Cuts"))
 (gr_line (start 112 101) (end 120 101) (stroke (width 0.1) (type default)) (layer "Edge.Cuts"))
 (segment (start 111.836 113.538) (end 113.792 113.538) (width 0.25) (layer "F.Cu") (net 2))
 (segment (start 110.236 113.538) (end 110.236 114.8842) (width 0.25) (layer "F.Cu") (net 4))
 (via (at 110.236 114.8842) (size 0.8) (drill 0.4) (layers "F.Cu" "B.Cu") (free yes) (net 4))
 (segment (start 120 104) (end 117.361 104) (width 0.25) (layer "F.Cu") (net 1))
 (segment (start 116.6368 104.775) (end 116.6368 112.3188) (width 0.25) (layer "F.Cu") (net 1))
 (segment (start 116.6876 104.7242) (end 116.6368 104.775) (width 0.25) (layer "F.Cu") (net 1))
 (segment (start 115.617 113.3386) (end 115.617 113.538) (width 0.25) (layer "F.Cu") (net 1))
 (segment (start 116.6368 112.3188) (end 115.617 113.3386) (width 0.25) (layer "F.Cu") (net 1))
 (segment (start 117.361 104) (end 116.6876 104.6734) (width 0.25) (layer "F.Cu") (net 1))
 (segment (start 116.6876 104.6734) (end 116.6876 104.7242) (width 0.25) (layer "F.Cu") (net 1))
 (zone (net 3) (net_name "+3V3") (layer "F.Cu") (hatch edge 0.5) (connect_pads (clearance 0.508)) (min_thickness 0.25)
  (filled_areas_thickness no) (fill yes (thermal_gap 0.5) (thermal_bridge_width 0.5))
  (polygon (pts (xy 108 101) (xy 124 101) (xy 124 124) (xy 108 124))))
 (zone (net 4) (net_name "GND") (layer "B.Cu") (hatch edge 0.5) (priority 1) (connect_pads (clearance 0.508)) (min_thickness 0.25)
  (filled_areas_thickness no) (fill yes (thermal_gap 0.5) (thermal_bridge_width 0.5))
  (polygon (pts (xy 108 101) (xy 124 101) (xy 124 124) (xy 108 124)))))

